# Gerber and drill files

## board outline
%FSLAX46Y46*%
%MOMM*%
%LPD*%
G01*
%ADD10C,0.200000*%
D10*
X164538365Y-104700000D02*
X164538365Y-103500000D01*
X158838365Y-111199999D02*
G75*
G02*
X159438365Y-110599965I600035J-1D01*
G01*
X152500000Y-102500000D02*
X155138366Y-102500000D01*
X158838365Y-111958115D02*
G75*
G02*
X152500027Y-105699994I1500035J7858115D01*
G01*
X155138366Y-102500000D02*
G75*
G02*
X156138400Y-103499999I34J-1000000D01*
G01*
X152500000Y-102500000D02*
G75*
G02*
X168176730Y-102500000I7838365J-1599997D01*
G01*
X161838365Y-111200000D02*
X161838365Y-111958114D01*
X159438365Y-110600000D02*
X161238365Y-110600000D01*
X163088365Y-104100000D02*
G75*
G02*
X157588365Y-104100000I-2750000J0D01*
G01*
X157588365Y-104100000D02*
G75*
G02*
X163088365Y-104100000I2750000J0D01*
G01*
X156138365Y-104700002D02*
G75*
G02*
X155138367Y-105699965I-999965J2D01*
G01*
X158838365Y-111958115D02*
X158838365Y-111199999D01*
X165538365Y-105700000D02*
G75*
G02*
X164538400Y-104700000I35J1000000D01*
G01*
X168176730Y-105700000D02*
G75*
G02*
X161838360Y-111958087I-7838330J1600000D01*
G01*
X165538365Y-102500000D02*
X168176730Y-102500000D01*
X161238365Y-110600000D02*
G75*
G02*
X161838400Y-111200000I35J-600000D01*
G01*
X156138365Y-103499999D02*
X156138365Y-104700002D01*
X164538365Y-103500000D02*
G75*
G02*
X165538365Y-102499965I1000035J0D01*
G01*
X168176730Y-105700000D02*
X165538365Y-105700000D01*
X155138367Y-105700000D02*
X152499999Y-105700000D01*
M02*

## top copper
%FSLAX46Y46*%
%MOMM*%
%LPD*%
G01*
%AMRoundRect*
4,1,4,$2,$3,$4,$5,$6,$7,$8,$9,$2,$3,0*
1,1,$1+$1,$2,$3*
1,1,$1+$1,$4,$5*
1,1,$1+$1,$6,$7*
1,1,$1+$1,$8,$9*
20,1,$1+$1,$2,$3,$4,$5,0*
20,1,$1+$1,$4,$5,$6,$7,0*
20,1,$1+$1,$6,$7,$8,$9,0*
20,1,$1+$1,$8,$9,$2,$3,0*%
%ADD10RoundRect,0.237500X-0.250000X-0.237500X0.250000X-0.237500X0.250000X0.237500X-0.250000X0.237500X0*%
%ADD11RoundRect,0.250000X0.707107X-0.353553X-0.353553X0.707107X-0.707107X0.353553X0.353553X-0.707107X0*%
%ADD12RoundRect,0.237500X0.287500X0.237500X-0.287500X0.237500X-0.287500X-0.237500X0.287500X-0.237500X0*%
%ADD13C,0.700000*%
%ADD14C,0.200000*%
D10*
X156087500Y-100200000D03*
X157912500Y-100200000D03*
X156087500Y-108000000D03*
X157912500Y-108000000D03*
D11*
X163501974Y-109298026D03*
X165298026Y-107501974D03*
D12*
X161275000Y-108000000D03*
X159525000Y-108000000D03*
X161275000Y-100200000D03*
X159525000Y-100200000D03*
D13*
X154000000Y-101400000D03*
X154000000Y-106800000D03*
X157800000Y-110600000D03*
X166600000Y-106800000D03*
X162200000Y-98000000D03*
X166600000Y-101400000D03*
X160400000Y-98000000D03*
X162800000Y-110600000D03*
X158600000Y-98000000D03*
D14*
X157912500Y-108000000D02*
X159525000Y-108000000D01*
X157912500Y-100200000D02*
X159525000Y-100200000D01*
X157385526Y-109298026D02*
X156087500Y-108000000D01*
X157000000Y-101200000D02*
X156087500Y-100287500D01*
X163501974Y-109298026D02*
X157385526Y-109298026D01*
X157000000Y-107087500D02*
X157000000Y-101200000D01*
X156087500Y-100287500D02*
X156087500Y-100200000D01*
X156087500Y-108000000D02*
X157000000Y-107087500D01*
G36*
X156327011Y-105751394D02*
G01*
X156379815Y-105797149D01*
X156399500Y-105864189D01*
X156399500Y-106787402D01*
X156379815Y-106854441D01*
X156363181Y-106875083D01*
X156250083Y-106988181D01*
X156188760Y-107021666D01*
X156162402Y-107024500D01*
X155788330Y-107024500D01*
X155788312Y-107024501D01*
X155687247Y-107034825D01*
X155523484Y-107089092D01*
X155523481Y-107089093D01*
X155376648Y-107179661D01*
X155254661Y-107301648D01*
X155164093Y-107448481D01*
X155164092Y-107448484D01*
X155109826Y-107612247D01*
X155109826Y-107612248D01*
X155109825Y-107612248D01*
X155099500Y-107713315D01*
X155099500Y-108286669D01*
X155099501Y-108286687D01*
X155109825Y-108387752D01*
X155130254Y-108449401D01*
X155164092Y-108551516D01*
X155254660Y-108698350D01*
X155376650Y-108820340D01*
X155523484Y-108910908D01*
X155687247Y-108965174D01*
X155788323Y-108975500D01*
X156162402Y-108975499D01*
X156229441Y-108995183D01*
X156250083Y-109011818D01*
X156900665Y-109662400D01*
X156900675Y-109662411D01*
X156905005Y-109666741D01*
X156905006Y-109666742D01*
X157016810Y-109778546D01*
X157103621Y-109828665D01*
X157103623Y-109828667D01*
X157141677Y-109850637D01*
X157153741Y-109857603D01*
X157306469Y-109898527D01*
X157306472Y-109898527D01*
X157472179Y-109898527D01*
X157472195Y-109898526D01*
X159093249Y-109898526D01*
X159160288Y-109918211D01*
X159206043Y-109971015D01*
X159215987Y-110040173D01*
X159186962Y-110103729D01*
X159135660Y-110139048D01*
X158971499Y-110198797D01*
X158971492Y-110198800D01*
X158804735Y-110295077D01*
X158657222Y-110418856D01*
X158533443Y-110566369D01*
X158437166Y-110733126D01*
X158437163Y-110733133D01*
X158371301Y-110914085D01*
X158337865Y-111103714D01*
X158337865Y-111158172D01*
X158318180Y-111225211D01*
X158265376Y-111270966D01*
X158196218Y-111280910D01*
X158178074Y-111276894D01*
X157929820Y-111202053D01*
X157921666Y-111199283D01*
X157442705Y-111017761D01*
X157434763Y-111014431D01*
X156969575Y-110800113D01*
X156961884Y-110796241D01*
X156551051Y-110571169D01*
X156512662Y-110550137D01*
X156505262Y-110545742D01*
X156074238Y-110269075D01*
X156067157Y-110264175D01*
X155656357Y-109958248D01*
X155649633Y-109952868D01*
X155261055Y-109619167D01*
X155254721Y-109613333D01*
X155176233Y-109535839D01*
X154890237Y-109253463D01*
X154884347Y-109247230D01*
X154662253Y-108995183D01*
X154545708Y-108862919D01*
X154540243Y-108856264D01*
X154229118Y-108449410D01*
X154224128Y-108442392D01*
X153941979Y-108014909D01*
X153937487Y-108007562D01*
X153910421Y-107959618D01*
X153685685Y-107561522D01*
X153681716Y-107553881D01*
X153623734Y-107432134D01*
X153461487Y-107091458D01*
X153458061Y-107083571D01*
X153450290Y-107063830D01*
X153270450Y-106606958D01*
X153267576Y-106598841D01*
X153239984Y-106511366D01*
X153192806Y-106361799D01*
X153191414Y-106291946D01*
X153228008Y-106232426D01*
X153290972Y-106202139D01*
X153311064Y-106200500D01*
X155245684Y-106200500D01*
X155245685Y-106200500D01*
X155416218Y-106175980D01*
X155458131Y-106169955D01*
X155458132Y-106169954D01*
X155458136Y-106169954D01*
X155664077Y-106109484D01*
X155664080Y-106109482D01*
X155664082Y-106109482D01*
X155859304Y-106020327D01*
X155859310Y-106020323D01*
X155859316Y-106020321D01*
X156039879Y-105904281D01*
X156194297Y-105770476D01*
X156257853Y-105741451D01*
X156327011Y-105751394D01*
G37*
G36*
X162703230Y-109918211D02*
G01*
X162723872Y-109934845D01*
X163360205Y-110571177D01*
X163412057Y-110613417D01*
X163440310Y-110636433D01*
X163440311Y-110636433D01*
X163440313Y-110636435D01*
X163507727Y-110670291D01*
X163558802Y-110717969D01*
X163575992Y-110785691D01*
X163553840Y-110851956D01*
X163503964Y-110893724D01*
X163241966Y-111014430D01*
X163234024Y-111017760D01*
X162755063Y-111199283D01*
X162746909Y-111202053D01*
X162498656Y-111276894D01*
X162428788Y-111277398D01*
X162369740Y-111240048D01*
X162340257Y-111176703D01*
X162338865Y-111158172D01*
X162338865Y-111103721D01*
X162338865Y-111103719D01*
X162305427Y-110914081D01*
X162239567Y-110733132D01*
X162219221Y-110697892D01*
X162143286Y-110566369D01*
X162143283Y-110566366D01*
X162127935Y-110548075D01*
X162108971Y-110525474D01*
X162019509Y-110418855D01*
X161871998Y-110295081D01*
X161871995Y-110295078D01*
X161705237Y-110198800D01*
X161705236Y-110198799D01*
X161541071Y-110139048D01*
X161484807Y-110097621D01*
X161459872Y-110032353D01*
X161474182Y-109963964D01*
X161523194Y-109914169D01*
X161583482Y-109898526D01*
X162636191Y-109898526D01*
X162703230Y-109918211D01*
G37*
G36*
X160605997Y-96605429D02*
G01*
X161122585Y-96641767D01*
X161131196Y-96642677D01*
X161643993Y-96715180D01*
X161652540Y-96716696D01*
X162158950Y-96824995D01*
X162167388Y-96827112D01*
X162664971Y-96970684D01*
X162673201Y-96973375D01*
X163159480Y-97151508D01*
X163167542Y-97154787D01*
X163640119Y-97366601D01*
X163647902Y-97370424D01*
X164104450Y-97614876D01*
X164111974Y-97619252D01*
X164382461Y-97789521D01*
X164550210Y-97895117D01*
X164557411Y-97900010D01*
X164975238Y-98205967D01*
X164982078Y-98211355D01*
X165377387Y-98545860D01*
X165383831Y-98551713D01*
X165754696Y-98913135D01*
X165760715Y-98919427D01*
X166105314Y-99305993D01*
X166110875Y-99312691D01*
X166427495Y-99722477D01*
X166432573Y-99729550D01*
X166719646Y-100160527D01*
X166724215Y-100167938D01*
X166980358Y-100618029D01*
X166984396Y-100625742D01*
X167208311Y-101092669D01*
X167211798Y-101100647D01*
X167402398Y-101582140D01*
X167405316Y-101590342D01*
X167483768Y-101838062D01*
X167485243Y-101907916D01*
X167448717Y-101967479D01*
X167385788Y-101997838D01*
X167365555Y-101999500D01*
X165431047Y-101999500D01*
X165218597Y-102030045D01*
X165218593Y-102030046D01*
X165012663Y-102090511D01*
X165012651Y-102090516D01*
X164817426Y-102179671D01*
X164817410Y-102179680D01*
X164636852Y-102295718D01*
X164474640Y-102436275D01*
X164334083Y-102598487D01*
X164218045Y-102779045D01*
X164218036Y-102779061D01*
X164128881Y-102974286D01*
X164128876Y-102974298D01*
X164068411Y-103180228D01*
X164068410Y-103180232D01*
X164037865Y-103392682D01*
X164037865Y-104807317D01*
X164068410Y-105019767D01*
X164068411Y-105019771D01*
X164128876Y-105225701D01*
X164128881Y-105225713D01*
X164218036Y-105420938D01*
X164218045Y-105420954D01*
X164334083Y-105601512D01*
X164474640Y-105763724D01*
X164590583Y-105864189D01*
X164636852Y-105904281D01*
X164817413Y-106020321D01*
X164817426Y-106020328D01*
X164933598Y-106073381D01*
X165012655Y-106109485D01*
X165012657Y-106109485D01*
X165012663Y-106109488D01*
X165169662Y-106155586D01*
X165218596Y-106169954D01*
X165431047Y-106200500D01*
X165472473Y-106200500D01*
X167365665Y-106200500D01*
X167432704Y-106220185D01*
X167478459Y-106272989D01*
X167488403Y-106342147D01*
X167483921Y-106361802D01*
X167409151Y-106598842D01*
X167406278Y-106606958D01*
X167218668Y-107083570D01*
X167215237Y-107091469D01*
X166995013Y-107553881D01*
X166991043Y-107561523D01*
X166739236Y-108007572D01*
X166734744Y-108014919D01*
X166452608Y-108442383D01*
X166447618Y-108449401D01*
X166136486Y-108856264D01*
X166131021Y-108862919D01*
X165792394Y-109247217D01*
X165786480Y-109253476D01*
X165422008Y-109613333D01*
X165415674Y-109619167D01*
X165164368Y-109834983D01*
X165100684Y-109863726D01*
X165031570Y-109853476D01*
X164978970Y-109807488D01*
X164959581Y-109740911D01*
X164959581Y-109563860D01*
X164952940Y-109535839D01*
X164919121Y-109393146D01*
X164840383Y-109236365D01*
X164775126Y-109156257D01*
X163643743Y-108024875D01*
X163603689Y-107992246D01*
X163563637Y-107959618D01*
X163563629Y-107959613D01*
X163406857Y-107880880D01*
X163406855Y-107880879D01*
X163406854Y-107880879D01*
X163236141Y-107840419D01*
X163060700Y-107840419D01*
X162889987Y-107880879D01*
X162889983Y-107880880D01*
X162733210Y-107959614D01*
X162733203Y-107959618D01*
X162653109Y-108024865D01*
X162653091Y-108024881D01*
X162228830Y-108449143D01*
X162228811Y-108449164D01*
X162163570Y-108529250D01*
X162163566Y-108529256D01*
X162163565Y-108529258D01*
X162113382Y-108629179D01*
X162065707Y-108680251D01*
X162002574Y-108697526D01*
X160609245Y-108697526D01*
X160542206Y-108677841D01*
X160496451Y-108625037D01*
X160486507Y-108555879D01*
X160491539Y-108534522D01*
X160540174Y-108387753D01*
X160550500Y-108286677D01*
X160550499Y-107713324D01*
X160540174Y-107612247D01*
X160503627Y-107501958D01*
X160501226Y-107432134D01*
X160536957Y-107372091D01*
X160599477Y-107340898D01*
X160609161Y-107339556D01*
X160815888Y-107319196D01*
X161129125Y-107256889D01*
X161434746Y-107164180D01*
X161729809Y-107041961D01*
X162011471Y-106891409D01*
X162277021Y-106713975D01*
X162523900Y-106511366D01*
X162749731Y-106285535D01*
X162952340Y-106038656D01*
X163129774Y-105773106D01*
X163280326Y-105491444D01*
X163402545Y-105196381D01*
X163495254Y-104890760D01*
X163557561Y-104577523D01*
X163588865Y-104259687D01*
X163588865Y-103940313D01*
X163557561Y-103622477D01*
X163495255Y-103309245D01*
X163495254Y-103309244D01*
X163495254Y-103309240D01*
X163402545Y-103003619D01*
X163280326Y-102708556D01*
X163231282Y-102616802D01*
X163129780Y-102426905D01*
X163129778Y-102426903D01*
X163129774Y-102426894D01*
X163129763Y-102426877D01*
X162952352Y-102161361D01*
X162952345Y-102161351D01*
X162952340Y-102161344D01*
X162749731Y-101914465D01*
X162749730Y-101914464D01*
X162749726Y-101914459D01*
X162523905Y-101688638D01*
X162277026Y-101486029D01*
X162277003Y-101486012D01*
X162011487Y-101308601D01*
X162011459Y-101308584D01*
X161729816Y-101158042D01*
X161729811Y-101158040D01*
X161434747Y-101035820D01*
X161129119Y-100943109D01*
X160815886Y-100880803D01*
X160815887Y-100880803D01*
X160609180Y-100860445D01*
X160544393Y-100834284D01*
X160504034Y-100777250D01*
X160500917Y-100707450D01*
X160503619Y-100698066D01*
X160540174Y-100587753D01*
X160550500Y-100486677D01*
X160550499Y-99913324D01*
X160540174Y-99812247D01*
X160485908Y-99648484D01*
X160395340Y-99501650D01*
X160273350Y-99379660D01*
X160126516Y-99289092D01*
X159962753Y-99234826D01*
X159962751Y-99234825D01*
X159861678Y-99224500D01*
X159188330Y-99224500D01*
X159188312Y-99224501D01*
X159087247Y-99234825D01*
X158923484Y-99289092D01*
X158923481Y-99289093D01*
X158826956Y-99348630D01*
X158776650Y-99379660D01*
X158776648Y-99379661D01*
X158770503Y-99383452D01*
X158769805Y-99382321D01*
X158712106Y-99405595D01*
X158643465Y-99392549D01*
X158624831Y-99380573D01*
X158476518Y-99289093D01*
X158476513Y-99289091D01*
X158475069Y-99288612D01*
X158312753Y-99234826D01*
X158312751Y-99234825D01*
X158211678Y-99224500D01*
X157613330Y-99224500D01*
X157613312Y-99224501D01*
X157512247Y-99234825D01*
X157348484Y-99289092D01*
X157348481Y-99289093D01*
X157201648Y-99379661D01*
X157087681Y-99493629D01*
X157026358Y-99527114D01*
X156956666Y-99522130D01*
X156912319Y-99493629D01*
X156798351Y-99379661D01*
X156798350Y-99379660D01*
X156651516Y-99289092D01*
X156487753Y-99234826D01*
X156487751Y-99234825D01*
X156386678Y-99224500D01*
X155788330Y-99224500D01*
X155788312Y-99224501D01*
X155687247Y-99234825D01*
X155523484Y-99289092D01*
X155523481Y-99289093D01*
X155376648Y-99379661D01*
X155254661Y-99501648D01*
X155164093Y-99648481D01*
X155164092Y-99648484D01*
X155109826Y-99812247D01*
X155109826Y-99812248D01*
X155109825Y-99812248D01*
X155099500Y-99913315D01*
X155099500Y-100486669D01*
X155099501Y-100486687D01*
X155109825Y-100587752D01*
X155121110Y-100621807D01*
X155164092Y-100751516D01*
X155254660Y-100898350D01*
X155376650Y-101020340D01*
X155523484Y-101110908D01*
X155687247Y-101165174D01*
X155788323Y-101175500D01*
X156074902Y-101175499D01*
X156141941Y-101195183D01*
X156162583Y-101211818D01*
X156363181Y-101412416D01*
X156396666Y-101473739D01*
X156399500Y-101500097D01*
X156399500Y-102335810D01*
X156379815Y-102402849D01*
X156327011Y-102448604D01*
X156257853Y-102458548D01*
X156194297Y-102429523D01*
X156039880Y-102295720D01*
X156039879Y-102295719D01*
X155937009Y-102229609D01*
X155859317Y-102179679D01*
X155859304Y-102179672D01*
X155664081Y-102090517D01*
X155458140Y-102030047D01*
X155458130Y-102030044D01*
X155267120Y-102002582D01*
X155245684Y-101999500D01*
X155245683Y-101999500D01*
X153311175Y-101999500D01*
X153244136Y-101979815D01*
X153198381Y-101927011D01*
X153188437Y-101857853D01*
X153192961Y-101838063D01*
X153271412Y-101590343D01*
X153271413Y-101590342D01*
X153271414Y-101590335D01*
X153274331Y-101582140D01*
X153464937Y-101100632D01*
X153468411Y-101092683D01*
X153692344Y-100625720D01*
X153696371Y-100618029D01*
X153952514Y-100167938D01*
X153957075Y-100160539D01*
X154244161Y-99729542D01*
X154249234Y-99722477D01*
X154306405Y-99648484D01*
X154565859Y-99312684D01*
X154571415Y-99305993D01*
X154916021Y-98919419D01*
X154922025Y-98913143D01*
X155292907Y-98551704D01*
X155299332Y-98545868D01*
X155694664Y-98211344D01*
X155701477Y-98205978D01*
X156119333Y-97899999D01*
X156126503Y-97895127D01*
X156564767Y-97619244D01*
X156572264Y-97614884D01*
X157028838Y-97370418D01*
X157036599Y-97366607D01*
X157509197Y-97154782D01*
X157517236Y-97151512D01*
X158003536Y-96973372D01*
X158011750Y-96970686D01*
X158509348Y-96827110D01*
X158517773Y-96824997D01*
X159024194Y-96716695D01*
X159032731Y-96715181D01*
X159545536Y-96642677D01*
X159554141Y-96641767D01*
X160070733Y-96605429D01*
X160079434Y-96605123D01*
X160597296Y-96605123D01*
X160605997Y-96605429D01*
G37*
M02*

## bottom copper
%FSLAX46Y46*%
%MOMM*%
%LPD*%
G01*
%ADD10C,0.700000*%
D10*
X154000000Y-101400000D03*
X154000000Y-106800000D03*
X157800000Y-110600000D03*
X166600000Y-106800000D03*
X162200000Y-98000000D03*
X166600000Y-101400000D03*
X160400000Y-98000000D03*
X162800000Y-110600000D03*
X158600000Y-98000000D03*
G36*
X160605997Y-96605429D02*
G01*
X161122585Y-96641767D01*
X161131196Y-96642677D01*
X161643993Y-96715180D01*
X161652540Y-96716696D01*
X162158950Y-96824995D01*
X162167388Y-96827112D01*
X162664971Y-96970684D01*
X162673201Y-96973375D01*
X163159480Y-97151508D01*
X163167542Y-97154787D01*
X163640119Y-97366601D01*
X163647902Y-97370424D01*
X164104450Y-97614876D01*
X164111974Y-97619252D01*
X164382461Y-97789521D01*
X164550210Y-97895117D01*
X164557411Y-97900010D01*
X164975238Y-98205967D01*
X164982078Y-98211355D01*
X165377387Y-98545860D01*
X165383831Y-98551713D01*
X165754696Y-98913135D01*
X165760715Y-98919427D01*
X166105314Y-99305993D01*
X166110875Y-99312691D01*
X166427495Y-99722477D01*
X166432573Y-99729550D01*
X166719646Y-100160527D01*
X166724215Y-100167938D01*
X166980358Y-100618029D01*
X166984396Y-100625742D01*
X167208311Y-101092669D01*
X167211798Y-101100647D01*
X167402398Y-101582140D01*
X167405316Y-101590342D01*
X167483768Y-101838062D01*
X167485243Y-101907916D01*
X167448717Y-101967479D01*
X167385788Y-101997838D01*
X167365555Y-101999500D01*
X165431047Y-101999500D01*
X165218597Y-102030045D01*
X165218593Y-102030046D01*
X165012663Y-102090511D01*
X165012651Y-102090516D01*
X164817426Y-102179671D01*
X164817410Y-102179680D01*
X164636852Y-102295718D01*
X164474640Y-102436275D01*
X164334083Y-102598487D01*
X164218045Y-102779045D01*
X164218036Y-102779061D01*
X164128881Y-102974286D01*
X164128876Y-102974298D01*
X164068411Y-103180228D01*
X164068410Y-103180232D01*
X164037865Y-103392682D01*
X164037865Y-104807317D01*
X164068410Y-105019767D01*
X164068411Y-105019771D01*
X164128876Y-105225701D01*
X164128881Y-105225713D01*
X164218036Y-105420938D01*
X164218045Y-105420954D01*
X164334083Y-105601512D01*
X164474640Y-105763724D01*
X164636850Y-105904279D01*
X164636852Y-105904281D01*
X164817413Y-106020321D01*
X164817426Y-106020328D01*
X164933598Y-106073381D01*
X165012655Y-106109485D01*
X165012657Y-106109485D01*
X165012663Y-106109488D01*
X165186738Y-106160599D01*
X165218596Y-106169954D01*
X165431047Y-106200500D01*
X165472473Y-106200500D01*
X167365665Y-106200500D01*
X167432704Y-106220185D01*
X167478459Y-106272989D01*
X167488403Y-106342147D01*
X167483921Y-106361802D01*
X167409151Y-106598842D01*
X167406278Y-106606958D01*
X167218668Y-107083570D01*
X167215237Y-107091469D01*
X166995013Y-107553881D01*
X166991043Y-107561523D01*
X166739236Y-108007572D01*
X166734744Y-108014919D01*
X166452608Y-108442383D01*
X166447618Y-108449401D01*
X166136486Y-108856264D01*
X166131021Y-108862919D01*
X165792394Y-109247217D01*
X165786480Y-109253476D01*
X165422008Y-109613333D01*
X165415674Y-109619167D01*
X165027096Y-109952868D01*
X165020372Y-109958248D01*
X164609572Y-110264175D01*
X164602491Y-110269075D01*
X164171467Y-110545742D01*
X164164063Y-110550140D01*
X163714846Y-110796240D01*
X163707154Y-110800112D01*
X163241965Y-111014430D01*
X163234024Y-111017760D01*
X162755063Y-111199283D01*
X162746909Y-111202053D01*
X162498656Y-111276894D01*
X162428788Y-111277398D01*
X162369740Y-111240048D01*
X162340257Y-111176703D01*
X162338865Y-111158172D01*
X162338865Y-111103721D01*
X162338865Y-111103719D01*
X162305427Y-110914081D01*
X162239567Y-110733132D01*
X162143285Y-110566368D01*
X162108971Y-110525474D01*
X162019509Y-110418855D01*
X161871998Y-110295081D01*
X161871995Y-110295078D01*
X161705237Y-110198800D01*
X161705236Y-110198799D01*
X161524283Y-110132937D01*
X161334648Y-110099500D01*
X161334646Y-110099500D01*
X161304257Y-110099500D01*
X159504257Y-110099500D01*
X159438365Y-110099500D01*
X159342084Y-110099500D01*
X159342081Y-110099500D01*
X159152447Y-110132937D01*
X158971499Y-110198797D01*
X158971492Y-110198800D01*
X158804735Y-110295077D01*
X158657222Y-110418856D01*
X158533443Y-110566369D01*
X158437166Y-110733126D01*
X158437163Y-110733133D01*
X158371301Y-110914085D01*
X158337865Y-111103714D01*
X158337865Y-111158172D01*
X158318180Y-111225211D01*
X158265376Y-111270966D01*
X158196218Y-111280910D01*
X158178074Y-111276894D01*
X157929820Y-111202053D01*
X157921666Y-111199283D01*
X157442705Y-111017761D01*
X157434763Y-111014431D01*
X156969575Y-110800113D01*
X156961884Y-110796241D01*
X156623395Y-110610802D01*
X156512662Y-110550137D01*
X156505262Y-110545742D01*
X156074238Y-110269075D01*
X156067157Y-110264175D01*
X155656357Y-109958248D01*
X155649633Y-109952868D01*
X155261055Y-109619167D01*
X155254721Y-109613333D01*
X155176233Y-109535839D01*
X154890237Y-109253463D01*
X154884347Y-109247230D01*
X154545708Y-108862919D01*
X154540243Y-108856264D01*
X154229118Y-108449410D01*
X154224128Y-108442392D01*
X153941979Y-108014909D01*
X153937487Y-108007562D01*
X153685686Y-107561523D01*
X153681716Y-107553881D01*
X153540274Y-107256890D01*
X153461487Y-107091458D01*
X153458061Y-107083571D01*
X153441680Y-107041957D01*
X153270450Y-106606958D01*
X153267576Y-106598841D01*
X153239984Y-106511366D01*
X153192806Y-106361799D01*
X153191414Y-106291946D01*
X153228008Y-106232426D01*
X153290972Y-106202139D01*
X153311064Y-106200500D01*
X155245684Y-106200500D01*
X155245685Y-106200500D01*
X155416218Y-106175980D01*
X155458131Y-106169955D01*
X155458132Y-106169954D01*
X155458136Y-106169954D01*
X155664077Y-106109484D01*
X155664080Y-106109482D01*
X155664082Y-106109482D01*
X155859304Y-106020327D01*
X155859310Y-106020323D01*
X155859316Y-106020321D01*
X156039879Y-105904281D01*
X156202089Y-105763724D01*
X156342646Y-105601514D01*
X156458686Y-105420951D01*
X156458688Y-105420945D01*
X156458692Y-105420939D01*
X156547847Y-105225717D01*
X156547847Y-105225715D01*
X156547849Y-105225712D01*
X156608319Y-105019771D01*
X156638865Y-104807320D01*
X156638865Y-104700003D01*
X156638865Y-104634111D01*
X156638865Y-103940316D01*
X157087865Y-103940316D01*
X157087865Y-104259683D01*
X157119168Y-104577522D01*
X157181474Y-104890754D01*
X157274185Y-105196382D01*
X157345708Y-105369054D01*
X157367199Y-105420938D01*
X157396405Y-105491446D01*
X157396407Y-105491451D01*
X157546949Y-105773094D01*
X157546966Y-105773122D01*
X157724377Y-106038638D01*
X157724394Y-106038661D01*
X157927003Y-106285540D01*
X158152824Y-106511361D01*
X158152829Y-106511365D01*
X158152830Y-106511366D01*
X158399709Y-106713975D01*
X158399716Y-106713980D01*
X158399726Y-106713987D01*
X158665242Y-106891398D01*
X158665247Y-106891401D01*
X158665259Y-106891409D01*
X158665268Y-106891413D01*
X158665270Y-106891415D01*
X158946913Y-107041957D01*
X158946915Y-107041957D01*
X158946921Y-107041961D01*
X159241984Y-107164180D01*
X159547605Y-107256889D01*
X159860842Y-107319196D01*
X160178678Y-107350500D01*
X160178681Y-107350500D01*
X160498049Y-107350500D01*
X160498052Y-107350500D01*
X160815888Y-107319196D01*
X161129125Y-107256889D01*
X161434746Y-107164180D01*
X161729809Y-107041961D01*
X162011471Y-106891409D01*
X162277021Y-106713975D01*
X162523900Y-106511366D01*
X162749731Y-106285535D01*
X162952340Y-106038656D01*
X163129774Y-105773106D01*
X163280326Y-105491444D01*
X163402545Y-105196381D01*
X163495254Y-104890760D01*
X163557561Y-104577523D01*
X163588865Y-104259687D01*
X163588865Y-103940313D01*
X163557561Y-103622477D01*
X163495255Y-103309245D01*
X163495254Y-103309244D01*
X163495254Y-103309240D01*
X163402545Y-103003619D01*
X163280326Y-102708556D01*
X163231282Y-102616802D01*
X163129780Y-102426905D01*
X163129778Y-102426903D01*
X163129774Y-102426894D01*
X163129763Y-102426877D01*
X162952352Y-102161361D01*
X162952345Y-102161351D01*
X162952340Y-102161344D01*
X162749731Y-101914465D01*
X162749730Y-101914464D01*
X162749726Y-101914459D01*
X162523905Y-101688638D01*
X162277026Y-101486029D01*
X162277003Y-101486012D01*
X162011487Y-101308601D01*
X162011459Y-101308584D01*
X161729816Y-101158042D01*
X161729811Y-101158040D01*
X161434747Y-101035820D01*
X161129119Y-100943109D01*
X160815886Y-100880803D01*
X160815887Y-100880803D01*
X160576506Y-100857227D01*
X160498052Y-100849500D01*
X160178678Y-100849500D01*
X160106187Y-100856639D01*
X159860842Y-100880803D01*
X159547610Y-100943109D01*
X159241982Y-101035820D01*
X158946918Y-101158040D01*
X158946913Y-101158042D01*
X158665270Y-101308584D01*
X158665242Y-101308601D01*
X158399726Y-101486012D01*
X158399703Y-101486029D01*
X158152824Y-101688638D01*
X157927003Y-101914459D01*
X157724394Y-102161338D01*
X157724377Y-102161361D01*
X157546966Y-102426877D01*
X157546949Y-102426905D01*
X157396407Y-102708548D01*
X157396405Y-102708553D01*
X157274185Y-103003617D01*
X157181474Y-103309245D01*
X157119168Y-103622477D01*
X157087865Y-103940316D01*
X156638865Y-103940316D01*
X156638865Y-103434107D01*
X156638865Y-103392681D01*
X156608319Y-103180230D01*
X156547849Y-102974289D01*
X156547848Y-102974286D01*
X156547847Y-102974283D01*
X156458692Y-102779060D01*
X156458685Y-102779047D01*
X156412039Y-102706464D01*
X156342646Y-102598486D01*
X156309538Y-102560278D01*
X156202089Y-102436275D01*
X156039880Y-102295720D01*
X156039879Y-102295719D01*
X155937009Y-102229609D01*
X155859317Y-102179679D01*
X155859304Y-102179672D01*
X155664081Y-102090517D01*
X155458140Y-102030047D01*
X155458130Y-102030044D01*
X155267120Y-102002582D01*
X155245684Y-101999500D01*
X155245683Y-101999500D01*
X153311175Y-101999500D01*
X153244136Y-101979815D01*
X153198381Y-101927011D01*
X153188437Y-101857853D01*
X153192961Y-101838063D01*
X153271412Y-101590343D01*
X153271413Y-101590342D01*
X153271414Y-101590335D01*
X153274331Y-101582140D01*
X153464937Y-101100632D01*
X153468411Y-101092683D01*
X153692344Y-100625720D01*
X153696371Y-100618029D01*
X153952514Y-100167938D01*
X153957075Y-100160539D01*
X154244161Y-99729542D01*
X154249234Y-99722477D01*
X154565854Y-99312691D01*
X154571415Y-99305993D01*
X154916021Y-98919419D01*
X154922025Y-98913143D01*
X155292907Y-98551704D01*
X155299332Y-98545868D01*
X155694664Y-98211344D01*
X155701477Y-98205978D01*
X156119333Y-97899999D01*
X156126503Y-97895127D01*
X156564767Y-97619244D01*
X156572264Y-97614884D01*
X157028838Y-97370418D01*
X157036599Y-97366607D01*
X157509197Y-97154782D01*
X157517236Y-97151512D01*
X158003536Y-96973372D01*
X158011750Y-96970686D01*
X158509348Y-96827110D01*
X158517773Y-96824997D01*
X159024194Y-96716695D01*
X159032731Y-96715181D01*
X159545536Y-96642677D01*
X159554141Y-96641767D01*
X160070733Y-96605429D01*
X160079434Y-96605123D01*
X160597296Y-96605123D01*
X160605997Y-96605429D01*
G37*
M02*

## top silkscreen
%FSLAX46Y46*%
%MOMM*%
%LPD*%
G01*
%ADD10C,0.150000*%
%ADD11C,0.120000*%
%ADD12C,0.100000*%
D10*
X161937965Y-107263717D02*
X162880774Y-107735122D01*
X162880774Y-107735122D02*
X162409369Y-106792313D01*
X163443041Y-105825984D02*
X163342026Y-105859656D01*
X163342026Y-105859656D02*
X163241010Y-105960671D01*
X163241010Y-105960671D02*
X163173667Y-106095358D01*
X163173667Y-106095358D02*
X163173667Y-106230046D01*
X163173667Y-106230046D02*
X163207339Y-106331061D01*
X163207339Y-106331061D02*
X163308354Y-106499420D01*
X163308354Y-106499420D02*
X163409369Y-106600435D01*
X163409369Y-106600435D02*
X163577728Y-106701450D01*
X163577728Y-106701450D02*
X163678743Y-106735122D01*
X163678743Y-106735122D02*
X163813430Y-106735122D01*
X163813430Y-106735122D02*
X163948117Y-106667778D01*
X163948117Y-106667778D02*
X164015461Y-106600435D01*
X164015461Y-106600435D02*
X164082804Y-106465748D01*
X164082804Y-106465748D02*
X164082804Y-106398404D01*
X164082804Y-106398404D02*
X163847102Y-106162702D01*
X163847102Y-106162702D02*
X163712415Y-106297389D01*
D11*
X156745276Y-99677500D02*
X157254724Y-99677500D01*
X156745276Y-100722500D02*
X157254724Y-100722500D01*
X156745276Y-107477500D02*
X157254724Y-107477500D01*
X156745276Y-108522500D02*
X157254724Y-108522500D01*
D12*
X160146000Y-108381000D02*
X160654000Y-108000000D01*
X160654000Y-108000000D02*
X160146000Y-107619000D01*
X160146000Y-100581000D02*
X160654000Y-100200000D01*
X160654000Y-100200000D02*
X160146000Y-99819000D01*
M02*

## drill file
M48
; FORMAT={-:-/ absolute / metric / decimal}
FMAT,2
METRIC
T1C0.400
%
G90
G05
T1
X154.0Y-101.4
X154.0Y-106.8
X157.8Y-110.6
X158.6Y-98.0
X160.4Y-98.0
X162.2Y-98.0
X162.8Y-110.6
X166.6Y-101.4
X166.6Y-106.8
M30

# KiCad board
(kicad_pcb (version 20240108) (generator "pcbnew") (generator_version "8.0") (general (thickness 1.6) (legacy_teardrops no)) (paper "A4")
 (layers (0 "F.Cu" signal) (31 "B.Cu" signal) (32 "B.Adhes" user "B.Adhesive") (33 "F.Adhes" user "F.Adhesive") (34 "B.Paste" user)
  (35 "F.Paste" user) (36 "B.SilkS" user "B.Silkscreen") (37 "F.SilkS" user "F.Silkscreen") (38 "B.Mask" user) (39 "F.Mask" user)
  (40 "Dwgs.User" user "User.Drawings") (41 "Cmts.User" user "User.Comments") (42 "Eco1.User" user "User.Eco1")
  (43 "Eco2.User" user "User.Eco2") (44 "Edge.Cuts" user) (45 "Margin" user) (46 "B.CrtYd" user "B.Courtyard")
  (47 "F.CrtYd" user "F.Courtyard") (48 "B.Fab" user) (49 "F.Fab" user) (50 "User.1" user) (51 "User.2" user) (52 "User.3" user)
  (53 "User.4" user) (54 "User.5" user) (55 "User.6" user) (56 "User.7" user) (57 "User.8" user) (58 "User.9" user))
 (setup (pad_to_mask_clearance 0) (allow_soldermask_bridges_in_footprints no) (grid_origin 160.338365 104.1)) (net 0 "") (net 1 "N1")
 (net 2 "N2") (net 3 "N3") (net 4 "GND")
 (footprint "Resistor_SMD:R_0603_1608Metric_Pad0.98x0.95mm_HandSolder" (layer "F.Cu") (at 157 100.2)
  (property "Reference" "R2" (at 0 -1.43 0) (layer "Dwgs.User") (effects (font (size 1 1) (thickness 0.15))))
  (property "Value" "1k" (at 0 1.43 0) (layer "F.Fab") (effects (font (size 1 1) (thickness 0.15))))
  (fp_line (start -0.254724 -0.5225) (end 0.254724 -0.5225) (stroke (width 0.12) (type solid)) (layer "F.SilkS"))
  (fp_line (start -0.254724 0.5225) (end 0.254724 0.5225) (stroke (width 0.12) (type solid)) (layer "F.SilkS"))
  (pad "1" smd roundrect (at -0.9125 0) (size 0.975 0.95) (layers "F.Cu" "F.Paste" "F.Mask") (roundrect_rratio 0.25) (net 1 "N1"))
  (pad "2" smd roundrect (at 0.9125 0) (size 0.975 0.95) (layers "F.Cu" "F.Paste" "F.Mask") (roundrect_rratio 0.25) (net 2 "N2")))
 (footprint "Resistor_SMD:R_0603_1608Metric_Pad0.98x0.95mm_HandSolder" (layer "F.Cu") (at 157 108)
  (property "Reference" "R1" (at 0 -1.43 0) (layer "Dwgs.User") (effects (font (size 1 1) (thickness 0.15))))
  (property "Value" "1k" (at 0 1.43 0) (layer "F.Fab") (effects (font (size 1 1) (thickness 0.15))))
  (fp_line (start -0.254724 -0.5225) (end 0.254724 -0.5225) (stroke (width 0.12) (type solid)) (layer "F.SilkS"))
  (fp_line (start -0.254724 0.5225) (end 0.254724 0.5225) (stroke (width 0.12) (type solid)) (layer "F.SilkS"))
  (pad "1" smd roundrect (at -0.9125 0) (size 0.975 0.95) (layers "F.Cu" "F.Paste" "F.Mask") (roundrect_rratio 0.25) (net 1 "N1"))
  (pad "2" smd roundrect (at 0.9125 0) (size 0.975 0.95) (layers "F.Cu" "F.Paste" "F.Mask") (roundrect_rratio 0.25) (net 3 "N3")))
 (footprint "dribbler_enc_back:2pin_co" (layer "F.Cu") (at 164.4 108.4 45)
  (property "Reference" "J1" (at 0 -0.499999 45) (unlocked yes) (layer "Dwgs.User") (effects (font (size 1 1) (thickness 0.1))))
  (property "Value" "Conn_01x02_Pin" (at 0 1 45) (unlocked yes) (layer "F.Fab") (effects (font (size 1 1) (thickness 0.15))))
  (pad "1" smd roundrect (at -1.270001 0 135) (size 2 1) (layers "F.Cu" "F.Paste" "F.Mask") (roundrect_rratio 0.25) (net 1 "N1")
   (thermal_bridge_angle 45))
  (pad "2" smd roundrect (at 1.270001 0 135) (size 2 1) (layers "F.Cu" "F.Paste" "F.Mask") (roundrect_rratio 0.25) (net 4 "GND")
   (thermal_bridge_angle 45)))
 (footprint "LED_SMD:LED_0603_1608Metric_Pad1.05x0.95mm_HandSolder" (layer "F.Cu") (at 160.4 108 180)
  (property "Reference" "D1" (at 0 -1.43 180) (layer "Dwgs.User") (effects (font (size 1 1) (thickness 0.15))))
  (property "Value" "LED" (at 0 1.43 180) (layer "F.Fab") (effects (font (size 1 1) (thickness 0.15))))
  (fp_line (start 0.254 -0.381) (end -0.254 0) (stroke (width 0.1) (type default)) (layer "F.SilkS"))
  (fp_line (start -0.254 0) (end 0.254 0.381) (stroke (width 0.1) (type default)) (layer "F.SilkS"))
  (pad "1" smd roundrect (at -0.875 0 180) (size 1.05 0.95) (layers "F.Cu" "F.Paste" "F.Mask") (roundrect_rratio 0.25) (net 4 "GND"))
  (pad "2" smd roundrect (at 0.875 0 180) (size 1.05 0.95) (layers "F.Cu" "F.Paste" "F.Mask") (roundrect_rratio 0.25) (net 3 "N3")))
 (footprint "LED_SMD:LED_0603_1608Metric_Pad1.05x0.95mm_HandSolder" (layer "F.Cu") (at 160.4 100.2 180)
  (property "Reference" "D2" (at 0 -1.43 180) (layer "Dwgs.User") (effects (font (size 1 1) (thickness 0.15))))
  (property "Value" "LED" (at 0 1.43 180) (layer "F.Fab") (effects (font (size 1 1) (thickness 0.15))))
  (fp_line (start 0.254 -0.381) (end -0.254 0) (stroke (width 0.1) (type default)) (layer "F.SilkS"))
  (fp_line (start -0.254 0) (end 0.254 0.381) (stroke (width 0.1) (type default)) (layer "F.SilkS"))
  (pad "1" smd roundrect (at -0.875 0 180) (size 1.05 0.95) (layers "F.Cu" "F.Paste" "F.Mask") (roundrect_rratio 0.25) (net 4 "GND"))
  (pad "2" smd roundrect (at 0.875 0 180) (size 1.05 0.95) (layers "F.Cu" "F.Paste" "F.Mask") (roundrect_rratio 0.25) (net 2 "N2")))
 (gr_line (start 164.538365 104.7) (end 164.538365 103.5) (stroke (width 0.2) (type default)) (layer "Edge.Cuts"))
 (gr_arc (start 158.838365 111.199999) (mid 159.014101 110.775736) (end 159.438365 110.6) (stroke (width 0.2) (type default))
  (layer "Edge.Cuts"))
 (gr_line (start 152.5 102.5) (end 155.138366 102.5) (stroke (width 0.2) (type default)) (layer "Edge.Cuts"))
 (gr_arc (start 158.838365 111.958115) (mid 154.717664 109.792778) (end 152.499999 105.7) (stroke (width 0.2) (type default))
  (layer "Edge.Cuts"))
 (gr_arc (start 155.138366 102.5) (mid 155.845472 102.792893) (end 156.138365 103.499999) (stroke (width 0.2) (type default))
  (layer "Edge.Cuts"))
 (gr_arc (start 152.5 102.5) (mid 160.338365 96.1) (end 168.17673 102.5) (stroke (width 0.2) (type default)) (layer "Edge.Cuts"))
 (gr_line (start 161.838365 111.2) (end 161.838365 111.958114) (stroke (width 0.2) (type default)) (layer "Edge.Cuts"))
 (gr_line (start 159.438365 110.6) (end 161.238365 110.6) (stroke (width 0.2) (type default)) (layer "Edge.Cuts"))
 (gr_circle (center 160.338365 104.1) (end 163.088365 104.1) (stroke (width 0.2) (type default)) (fill none) (layer "Edge.Cuts"))
 (gr_arc (start 156.138365 104.700002) (mid 155.845472 105.407107) (end 155.138367 105.7) (stroke (width 0.2) (type default))
  (layer "Edge.Cuts"))
 (gr_line (start 158.838365 111.958115) (end 158.838365 111.199999) (stroke (width 0.2) (type default)) (layer "Edge.Cuts"))
 (gr_arc (start 165.538365 105.7) (mid 164.831258 105.407107) (end 164.538365 104.7) (stroke (width 0.2) (type default)) (layer "Edge.Cuts"))
 (gr_arc (start 168.17673 105.7) (mid 165.959066 109.792778) (end 161.838365 111.958114) (stroke (width 0.2) (type default))
  (layer "Edge.Cuts"))
 (gr_line (start 165.538365 102.5) (end 168.17673 102.5) (stroke (width 0.2) (type default)) (layer "Edge.Cuts"))
 (gr_arc (start 161.238365 110.6) (mid 161.662629 110.775736) (end 161.838365 111.2) (stroke (width 0.2) (type default)) (layer "Edge.Cuts"))
 (gr_line (start 156.138365 103.499999) (end 156.138365 104.700002) (stroke (width 0.2) (type default)) (layer "Edge.Cuts"))
 (gr_arc (start 164.538365 103.5) (mid 164.831258 102.792893) (end 165.538365 102.5) (stroke (width 0.2) (type default)) (layer "Edge.Cuts"))
 (gr_line (start 168.17673 105.7) (end 165.538365 105.7) (stroke (width 0.2) (type default)) (layer "Edge.Cuts"))
 (gr_line (start 155.138367 105.7) (end 152.499999 105.7) (stroke (width 0.2) (type default)) (layer "Edge.Cuts"))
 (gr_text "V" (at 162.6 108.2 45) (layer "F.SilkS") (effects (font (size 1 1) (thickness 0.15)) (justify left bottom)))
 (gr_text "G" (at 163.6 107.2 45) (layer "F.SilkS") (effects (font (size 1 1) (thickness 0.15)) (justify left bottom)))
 (via (at 154 101.4) (size 0.7) (drill 0.4) (layers "F.Cu" "B.Cu") (free yes) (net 4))
 (via (at 154 106.8) (size 0.7) (drill 0.4) (layers "F.Cu" "B.Cu") (free yes) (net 4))
 (via (at 157.8 110.6) (size 0.7) (drill 0.4) (layers "F.Cu" "B.Cu") (free yes) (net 4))
 (via (at 166.6 106.8) (size 0.7) (drill 0.4) (layers "F.Cu" "B.Cu") (free yes) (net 4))
 (via (at 162.2 98) (size 0.7) (drill 0.4) (layers "F.Cu" "B.Cu") (free yes) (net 4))
 (via (at 166.6 101.4) (size 0.7) (drill 0.4) (layers "F.Cu" "B.Cu") (free yes) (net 4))
 (via (at 160.4 98) (size 0.7) (drill 0.4) (layers "F.Cu" "B.Cu") (free yes) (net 4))
 (via (at 162.8 110.6) (size 0.7) (drill 0.4) (layers "F.Cu" "B.Cu") (free yes) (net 4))
 (via (at 158.6 98) (size 0.7) (drill 0.4) (layers "F.Cu" "B.Cu") (free yes) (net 4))
 (segment (start 157.9125 108) (end 159.525 108) (width 0.2) (layer "F.Cu") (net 3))
 (segment (start 157.9125 100.2) (end 159.525 100.2) (width 0.2) (layer "F.Cu") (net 2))
 (segment (start 157.385526 109.298026) (end 156.0875 108) (width 0.2) (layer "F.Cu") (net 1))
 (segment (start 157 101.2) (end 156.0875 100.2875) (width 0.2) (layer "F.Cu") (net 1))
 (segment (start 163.501974 109.298026) (end 157.385526 109.298026) (width 0.2) (layer "F.Cu") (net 1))
 (segment (start 157 107.0875) (end 157 101.2) (width 0.2) (layer "F.Cu") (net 1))
 (segment (start 156.0875 100.2875) (end 156.0875 100.2) (width 0.2) (layer "F.Cu") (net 1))
 (segment (start 156.0875 108) (end 157 107.0875) (width 0.2) (layer "F.Cu") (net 1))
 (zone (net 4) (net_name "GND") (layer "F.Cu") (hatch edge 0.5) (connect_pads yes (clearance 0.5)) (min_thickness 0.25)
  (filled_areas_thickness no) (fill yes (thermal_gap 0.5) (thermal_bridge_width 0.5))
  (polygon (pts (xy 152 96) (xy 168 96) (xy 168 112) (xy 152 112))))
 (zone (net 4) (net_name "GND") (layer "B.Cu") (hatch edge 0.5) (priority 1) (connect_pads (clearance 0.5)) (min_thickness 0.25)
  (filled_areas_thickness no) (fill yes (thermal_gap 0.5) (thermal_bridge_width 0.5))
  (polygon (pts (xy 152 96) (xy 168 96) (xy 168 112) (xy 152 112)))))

